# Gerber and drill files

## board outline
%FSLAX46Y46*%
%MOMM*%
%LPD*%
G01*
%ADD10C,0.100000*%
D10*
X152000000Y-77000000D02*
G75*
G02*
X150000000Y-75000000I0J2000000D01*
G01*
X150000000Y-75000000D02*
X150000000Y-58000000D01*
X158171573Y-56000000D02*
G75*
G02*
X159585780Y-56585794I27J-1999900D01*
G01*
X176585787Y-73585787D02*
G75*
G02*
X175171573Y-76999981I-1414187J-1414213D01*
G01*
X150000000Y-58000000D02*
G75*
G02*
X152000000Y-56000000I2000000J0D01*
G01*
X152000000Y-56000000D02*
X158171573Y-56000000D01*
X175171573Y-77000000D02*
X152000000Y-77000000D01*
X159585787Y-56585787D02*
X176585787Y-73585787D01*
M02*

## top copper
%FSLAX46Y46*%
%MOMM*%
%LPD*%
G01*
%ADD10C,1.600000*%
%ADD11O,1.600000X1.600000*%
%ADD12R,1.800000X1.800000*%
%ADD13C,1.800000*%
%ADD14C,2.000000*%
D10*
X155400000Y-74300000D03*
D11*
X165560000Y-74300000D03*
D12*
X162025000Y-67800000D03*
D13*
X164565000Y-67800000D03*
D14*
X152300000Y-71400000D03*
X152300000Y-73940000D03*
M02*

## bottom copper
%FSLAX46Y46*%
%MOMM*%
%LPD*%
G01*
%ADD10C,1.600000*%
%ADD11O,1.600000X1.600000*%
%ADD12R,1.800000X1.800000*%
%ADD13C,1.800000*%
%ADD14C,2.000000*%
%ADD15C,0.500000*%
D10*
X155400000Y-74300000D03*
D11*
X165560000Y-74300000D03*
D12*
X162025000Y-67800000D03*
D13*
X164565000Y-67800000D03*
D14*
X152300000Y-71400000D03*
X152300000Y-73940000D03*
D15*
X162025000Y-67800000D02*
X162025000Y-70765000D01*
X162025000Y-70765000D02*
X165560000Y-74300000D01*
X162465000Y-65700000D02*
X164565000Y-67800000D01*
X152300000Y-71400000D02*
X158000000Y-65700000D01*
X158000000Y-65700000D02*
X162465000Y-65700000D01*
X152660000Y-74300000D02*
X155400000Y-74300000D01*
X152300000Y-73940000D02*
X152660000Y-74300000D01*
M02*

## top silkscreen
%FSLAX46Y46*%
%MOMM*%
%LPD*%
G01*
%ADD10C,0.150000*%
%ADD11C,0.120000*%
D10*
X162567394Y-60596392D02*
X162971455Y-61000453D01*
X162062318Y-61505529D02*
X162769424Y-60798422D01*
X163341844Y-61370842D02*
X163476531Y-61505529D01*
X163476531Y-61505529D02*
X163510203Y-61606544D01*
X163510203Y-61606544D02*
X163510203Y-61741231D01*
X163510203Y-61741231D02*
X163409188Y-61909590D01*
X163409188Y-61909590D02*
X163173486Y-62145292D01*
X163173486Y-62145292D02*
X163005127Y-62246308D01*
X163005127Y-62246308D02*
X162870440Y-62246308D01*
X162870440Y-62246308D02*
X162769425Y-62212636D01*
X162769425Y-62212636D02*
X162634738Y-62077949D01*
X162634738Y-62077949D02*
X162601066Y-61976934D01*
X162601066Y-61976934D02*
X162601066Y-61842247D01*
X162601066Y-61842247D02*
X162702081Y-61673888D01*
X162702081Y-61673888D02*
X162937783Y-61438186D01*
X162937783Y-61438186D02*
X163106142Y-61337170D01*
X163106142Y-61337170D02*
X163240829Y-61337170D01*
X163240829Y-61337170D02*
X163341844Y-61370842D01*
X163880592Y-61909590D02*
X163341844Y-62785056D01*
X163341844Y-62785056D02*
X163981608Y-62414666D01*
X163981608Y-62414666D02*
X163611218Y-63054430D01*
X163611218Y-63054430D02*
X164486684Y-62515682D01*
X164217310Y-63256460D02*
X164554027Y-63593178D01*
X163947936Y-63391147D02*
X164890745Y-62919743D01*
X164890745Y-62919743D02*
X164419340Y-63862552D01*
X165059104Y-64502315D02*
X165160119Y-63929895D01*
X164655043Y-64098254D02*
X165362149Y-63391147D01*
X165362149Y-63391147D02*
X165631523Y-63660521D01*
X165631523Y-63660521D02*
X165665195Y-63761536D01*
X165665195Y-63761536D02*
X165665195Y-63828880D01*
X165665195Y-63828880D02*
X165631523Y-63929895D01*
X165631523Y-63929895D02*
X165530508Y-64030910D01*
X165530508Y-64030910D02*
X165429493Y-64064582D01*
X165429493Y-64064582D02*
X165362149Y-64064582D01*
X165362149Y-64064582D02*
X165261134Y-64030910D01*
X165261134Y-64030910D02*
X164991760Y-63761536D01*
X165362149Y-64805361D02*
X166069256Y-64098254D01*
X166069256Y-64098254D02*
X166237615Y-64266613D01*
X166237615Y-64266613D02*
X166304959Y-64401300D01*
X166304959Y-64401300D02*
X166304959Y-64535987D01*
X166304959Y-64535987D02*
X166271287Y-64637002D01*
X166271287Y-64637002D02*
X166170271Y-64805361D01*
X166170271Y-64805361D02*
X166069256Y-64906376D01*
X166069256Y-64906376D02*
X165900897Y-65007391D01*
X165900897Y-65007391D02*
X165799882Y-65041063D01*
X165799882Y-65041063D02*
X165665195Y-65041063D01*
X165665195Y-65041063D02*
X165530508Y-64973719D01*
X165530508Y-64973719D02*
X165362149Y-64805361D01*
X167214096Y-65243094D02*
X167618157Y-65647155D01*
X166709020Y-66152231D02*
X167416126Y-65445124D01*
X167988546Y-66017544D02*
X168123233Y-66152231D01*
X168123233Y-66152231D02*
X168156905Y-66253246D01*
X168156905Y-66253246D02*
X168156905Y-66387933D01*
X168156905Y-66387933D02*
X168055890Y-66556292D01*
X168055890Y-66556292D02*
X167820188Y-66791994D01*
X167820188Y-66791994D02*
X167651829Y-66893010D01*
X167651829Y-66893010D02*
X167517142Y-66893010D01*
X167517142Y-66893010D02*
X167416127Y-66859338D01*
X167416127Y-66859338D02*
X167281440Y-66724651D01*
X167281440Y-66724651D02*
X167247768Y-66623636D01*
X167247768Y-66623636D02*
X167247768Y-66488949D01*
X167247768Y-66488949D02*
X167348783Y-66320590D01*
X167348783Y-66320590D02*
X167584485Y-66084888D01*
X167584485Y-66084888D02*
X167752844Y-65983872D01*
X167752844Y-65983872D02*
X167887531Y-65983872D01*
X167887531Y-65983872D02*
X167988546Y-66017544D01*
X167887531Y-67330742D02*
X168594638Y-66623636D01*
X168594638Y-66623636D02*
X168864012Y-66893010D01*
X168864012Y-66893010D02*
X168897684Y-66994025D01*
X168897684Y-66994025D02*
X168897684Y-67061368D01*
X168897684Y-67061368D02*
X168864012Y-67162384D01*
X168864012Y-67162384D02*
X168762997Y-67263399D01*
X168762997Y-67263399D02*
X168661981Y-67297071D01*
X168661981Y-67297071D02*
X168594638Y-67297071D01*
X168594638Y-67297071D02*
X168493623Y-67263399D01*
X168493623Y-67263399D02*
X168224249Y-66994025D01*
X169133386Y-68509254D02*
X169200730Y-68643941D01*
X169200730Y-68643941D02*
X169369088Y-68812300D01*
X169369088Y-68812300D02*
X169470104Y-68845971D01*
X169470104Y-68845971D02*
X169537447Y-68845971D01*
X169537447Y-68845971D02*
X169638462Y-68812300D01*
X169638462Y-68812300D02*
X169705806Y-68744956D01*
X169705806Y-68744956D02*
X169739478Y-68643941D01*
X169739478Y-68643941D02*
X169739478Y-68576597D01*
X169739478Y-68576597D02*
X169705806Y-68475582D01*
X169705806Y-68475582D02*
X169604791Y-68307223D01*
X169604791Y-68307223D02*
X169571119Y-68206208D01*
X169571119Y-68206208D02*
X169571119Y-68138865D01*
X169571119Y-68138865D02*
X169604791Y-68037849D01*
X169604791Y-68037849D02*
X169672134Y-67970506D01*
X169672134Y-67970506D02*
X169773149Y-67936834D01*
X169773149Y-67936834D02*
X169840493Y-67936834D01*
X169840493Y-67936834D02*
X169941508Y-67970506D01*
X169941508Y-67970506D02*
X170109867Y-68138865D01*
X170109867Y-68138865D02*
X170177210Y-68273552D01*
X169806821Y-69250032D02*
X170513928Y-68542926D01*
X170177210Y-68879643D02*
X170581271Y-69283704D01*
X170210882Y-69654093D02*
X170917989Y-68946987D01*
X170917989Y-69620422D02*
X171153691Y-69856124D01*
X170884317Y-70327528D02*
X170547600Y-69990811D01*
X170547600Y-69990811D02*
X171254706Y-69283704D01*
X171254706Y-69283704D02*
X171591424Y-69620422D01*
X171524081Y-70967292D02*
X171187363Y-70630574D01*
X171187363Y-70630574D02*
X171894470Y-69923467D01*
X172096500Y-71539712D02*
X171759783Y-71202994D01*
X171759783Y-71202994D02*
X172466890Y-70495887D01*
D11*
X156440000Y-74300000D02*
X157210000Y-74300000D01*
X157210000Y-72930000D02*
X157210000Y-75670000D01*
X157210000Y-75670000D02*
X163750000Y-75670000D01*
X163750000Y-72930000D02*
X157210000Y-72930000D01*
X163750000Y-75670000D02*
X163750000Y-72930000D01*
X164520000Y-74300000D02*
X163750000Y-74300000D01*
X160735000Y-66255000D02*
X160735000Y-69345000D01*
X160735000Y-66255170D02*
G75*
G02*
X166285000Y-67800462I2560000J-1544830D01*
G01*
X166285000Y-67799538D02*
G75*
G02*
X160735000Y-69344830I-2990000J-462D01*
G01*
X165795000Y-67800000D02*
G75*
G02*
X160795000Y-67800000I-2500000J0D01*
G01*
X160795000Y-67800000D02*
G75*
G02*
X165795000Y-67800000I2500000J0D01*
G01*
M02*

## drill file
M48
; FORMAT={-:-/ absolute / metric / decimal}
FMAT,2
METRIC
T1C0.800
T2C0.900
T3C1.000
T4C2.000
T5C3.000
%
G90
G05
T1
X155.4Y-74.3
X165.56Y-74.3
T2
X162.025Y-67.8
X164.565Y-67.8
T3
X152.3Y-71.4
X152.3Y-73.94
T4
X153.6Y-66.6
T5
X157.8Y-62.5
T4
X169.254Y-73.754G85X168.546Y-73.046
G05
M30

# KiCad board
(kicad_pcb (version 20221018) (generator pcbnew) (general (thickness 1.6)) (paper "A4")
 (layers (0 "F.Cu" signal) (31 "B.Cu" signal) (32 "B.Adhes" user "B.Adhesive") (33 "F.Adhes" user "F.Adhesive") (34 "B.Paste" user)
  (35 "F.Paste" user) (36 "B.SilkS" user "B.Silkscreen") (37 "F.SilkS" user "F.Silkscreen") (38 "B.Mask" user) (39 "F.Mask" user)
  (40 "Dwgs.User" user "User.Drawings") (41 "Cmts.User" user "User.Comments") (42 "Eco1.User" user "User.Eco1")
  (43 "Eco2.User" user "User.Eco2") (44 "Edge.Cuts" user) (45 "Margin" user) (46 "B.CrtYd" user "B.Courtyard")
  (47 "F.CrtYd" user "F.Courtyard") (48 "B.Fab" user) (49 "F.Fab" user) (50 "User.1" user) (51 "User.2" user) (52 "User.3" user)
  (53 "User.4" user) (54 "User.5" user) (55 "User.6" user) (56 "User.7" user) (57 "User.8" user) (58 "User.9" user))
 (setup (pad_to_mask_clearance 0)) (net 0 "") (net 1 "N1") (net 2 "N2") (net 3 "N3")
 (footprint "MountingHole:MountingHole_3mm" (layer "F.Cu") (at 157.8 62.5)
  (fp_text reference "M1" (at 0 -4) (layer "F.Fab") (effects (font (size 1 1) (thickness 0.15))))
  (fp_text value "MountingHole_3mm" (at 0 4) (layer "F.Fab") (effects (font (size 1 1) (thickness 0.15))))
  (pad "" np_thru_hole circle (at 0 0) (size 3 3) (drill 3) (layers "*.Cu" "*.Mask")))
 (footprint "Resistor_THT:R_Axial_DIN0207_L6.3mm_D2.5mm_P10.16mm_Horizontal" (layer "F.Cu") (at 155.4 74.3)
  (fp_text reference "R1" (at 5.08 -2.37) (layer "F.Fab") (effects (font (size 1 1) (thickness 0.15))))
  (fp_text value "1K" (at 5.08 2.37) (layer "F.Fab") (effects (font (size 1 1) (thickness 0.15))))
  (fp_line (start 1.04 0) (end 1.81 0) (stroke (width 0.12) (type solid)) (layer "F.SilkS"))
  (fp_line (start 1.81 -1.37) (end 1.81 1.37) (stroke (width 0.12) (type solid)) (layer "F.SilkS"))
  (fp_line (start 1.81 1.37) (end 8.35 1.37) (stroke (width 0.12) (type solid)) (layer "F.SilkS"))
  (fp_line (start 8.35 -1.37) (end 1.81 -1.37) (stroke (width 0.12) (type solid)) (layer "F.SilkS"))
  (fp_line (start 8.35 1.37) (end 8.35 -1.37) (stroke (width 0.12) (type solid)) (layer "F.SilkS"))
  (fp_line (start 9.12 0) (end 8.35 0) (stroke (width 0.12) (type solid)) (layer "F.SilkS"))
  (pad "1" thru_hole circle (at 0 0) (size 1.6 1.6) (drill 0.8) (layers "*.Cu" "*.Mask") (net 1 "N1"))
  (pad "2" thru_hole oval (at 10.16 0) (size 1.6 1.6) (drill 0.8) (layers "*.Cu" "*.Mask") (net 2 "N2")))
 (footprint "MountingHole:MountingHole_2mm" (layer "F.Cu") (at 168.9 73.4 135)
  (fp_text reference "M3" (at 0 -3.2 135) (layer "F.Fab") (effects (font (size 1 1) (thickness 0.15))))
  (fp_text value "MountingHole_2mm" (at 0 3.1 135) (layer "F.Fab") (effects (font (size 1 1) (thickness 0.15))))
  (pad "" np_thru_hole oval (at 0 0 135) (size 3 2) (drill oval 3 2) (layers "F&B.Cu" "*.Mask")))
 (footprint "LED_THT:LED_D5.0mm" (layer "F.Cu") (at 162.025 67.8)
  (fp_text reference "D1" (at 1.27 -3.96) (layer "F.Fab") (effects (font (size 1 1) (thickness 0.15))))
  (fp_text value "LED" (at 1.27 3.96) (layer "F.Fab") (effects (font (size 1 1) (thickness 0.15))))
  (fp_line (start -1.29 -1.545) (end -1.29 1.545) (stroke (width 0.12) (type solid)) (layer "F.SilkS"))
  (fp_arc (start -1.29 -1.54483) (mid 2.072002 -2.880433) (end 4.26 0.000462) (stroke (width 0.12) (type solid)) (layer "F.SilkS"))
  (fp_arc (start 4.26 -0.000462) (mid 2.072002 2.880433) (end -1.29 1.54483) (stroke (width 0.12) (type solid)) (layer "F.SilkS"))
  (fp_circle (center 1.27 0) (end 3.77 0) (stroke (width 0.12) (type solid)) (fill none) (layer "F.SilkS"))
  (pad "1" thru_hole rect (at 0 0) (size 1.8 1.8) (drill 0.9) (layers "*.Cu" "*.Mask") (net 2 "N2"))
  (pad "2" thru_hole circle (at 2.54 0) (size 1.8 1.8) (drill 0.9) (layers "*.Cu" "*.Mask") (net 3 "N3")))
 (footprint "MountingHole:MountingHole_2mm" (layer "F.Cu") (at 153.6 66.6)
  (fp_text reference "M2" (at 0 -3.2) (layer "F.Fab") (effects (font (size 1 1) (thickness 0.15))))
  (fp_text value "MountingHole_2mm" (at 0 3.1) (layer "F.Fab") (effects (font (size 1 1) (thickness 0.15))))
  (pad "" np_thru_hole circle (at 0 0) (size 2 2) (drill 2) (layers "*.Cu" "*.Mask")))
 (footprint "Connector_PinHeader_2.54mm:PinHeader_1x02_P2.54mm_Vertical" (layer "B.Cu") (at 152.3 71.4 180)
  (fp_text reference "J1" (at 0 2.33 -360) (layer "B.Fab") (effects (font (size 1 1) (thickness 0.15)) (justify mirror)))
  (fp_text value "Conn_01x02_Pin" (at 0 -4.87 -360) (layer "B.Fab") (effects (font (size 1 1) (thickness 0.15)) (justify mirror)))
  (pad "1" thru_hole circle (at 0 0 180) (size 2 2) (drill 1) (layers "*.Cu" "*.Mask") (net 3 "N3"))
  (pad "2" thru_hole circle (at 0 -2.54 180) (size 2 2) (drill 1) (layers "*.Cu" "*.Mask") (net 1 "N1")))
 (gr_arc (start 152 77) (mid 150.585786 76.414214) (end 150 75) (stroke (width 0.1) (type default)) (layer "Edge.Cuts"))
 (gr_line (start 150 75) (end 150 58) (stroke (width 0.1) (type default)) (layer "Edge.Cuts"))
 (gr_arc (start 158.171573 56) (mid 158.936946 56.152232) (end 159.585787 56.585787) (stroke (width 0.1) (type default)) (layer "Edge.Cuts"))
 (gr_arc (start 176.585787 73.585787) (mid 177.019332 75.765367) (end 175.171573 77) (stroke (width 0.1) (type default)) (layer "Edge.Cuts"))
 (gr_arc (start 150 58) (mid 150.585786 56.585786) (end 152 56) (stroke (width 0.1) (type default)) (layer "Edge.Cuts"))
 (gr_line (start 152 56) (end 158.171573 56) (stroke (width 0.1) (type default)) (layer "Edge.Cuts"))
 (gr_line (start 175.171573 77) (end 152 77) (stroke (width 0.1) (type default)) (layer "Edge.Cuts"))
 (gr_line (start 159.585787 56.585787) (end 176.585787 73.585787) (stroke (width 0.1) (type default)) (layer "Edge.Cuts"))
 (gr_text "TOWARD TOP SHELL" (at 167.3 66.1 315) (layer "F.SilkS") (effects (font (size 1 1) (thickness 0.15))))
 (segment (start 162.025 67.8) (end 162.025 70.765) (width 0.5) (layer "B.Cu") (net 2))
 (segment (start 162.025 70.765) (end 165.56 74.3) (width 0.5) (layer "B.Cu") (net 2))
 (segment (start 162.465 65.7) (end 164.565 67.8) (width 0.5) (layer "B.Cu") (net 3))
 (segment (start 152.3 71.4) (end 158 65.7) (width 0.5) (layer "B.Cu") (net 3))
 (segment (start 158 65.7) (end 162.465 65.7) (width 0.5) (layer "B.Cu") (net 3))
 (segment (start 152.66 74.3) (end 155.4 74.3) (width 0.5) (layer "B.Cu") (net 1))
 (segment (start 152.3 73.94) (end 152.66 74.3) (width 0.5) (layer "B.Cu") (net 1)))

